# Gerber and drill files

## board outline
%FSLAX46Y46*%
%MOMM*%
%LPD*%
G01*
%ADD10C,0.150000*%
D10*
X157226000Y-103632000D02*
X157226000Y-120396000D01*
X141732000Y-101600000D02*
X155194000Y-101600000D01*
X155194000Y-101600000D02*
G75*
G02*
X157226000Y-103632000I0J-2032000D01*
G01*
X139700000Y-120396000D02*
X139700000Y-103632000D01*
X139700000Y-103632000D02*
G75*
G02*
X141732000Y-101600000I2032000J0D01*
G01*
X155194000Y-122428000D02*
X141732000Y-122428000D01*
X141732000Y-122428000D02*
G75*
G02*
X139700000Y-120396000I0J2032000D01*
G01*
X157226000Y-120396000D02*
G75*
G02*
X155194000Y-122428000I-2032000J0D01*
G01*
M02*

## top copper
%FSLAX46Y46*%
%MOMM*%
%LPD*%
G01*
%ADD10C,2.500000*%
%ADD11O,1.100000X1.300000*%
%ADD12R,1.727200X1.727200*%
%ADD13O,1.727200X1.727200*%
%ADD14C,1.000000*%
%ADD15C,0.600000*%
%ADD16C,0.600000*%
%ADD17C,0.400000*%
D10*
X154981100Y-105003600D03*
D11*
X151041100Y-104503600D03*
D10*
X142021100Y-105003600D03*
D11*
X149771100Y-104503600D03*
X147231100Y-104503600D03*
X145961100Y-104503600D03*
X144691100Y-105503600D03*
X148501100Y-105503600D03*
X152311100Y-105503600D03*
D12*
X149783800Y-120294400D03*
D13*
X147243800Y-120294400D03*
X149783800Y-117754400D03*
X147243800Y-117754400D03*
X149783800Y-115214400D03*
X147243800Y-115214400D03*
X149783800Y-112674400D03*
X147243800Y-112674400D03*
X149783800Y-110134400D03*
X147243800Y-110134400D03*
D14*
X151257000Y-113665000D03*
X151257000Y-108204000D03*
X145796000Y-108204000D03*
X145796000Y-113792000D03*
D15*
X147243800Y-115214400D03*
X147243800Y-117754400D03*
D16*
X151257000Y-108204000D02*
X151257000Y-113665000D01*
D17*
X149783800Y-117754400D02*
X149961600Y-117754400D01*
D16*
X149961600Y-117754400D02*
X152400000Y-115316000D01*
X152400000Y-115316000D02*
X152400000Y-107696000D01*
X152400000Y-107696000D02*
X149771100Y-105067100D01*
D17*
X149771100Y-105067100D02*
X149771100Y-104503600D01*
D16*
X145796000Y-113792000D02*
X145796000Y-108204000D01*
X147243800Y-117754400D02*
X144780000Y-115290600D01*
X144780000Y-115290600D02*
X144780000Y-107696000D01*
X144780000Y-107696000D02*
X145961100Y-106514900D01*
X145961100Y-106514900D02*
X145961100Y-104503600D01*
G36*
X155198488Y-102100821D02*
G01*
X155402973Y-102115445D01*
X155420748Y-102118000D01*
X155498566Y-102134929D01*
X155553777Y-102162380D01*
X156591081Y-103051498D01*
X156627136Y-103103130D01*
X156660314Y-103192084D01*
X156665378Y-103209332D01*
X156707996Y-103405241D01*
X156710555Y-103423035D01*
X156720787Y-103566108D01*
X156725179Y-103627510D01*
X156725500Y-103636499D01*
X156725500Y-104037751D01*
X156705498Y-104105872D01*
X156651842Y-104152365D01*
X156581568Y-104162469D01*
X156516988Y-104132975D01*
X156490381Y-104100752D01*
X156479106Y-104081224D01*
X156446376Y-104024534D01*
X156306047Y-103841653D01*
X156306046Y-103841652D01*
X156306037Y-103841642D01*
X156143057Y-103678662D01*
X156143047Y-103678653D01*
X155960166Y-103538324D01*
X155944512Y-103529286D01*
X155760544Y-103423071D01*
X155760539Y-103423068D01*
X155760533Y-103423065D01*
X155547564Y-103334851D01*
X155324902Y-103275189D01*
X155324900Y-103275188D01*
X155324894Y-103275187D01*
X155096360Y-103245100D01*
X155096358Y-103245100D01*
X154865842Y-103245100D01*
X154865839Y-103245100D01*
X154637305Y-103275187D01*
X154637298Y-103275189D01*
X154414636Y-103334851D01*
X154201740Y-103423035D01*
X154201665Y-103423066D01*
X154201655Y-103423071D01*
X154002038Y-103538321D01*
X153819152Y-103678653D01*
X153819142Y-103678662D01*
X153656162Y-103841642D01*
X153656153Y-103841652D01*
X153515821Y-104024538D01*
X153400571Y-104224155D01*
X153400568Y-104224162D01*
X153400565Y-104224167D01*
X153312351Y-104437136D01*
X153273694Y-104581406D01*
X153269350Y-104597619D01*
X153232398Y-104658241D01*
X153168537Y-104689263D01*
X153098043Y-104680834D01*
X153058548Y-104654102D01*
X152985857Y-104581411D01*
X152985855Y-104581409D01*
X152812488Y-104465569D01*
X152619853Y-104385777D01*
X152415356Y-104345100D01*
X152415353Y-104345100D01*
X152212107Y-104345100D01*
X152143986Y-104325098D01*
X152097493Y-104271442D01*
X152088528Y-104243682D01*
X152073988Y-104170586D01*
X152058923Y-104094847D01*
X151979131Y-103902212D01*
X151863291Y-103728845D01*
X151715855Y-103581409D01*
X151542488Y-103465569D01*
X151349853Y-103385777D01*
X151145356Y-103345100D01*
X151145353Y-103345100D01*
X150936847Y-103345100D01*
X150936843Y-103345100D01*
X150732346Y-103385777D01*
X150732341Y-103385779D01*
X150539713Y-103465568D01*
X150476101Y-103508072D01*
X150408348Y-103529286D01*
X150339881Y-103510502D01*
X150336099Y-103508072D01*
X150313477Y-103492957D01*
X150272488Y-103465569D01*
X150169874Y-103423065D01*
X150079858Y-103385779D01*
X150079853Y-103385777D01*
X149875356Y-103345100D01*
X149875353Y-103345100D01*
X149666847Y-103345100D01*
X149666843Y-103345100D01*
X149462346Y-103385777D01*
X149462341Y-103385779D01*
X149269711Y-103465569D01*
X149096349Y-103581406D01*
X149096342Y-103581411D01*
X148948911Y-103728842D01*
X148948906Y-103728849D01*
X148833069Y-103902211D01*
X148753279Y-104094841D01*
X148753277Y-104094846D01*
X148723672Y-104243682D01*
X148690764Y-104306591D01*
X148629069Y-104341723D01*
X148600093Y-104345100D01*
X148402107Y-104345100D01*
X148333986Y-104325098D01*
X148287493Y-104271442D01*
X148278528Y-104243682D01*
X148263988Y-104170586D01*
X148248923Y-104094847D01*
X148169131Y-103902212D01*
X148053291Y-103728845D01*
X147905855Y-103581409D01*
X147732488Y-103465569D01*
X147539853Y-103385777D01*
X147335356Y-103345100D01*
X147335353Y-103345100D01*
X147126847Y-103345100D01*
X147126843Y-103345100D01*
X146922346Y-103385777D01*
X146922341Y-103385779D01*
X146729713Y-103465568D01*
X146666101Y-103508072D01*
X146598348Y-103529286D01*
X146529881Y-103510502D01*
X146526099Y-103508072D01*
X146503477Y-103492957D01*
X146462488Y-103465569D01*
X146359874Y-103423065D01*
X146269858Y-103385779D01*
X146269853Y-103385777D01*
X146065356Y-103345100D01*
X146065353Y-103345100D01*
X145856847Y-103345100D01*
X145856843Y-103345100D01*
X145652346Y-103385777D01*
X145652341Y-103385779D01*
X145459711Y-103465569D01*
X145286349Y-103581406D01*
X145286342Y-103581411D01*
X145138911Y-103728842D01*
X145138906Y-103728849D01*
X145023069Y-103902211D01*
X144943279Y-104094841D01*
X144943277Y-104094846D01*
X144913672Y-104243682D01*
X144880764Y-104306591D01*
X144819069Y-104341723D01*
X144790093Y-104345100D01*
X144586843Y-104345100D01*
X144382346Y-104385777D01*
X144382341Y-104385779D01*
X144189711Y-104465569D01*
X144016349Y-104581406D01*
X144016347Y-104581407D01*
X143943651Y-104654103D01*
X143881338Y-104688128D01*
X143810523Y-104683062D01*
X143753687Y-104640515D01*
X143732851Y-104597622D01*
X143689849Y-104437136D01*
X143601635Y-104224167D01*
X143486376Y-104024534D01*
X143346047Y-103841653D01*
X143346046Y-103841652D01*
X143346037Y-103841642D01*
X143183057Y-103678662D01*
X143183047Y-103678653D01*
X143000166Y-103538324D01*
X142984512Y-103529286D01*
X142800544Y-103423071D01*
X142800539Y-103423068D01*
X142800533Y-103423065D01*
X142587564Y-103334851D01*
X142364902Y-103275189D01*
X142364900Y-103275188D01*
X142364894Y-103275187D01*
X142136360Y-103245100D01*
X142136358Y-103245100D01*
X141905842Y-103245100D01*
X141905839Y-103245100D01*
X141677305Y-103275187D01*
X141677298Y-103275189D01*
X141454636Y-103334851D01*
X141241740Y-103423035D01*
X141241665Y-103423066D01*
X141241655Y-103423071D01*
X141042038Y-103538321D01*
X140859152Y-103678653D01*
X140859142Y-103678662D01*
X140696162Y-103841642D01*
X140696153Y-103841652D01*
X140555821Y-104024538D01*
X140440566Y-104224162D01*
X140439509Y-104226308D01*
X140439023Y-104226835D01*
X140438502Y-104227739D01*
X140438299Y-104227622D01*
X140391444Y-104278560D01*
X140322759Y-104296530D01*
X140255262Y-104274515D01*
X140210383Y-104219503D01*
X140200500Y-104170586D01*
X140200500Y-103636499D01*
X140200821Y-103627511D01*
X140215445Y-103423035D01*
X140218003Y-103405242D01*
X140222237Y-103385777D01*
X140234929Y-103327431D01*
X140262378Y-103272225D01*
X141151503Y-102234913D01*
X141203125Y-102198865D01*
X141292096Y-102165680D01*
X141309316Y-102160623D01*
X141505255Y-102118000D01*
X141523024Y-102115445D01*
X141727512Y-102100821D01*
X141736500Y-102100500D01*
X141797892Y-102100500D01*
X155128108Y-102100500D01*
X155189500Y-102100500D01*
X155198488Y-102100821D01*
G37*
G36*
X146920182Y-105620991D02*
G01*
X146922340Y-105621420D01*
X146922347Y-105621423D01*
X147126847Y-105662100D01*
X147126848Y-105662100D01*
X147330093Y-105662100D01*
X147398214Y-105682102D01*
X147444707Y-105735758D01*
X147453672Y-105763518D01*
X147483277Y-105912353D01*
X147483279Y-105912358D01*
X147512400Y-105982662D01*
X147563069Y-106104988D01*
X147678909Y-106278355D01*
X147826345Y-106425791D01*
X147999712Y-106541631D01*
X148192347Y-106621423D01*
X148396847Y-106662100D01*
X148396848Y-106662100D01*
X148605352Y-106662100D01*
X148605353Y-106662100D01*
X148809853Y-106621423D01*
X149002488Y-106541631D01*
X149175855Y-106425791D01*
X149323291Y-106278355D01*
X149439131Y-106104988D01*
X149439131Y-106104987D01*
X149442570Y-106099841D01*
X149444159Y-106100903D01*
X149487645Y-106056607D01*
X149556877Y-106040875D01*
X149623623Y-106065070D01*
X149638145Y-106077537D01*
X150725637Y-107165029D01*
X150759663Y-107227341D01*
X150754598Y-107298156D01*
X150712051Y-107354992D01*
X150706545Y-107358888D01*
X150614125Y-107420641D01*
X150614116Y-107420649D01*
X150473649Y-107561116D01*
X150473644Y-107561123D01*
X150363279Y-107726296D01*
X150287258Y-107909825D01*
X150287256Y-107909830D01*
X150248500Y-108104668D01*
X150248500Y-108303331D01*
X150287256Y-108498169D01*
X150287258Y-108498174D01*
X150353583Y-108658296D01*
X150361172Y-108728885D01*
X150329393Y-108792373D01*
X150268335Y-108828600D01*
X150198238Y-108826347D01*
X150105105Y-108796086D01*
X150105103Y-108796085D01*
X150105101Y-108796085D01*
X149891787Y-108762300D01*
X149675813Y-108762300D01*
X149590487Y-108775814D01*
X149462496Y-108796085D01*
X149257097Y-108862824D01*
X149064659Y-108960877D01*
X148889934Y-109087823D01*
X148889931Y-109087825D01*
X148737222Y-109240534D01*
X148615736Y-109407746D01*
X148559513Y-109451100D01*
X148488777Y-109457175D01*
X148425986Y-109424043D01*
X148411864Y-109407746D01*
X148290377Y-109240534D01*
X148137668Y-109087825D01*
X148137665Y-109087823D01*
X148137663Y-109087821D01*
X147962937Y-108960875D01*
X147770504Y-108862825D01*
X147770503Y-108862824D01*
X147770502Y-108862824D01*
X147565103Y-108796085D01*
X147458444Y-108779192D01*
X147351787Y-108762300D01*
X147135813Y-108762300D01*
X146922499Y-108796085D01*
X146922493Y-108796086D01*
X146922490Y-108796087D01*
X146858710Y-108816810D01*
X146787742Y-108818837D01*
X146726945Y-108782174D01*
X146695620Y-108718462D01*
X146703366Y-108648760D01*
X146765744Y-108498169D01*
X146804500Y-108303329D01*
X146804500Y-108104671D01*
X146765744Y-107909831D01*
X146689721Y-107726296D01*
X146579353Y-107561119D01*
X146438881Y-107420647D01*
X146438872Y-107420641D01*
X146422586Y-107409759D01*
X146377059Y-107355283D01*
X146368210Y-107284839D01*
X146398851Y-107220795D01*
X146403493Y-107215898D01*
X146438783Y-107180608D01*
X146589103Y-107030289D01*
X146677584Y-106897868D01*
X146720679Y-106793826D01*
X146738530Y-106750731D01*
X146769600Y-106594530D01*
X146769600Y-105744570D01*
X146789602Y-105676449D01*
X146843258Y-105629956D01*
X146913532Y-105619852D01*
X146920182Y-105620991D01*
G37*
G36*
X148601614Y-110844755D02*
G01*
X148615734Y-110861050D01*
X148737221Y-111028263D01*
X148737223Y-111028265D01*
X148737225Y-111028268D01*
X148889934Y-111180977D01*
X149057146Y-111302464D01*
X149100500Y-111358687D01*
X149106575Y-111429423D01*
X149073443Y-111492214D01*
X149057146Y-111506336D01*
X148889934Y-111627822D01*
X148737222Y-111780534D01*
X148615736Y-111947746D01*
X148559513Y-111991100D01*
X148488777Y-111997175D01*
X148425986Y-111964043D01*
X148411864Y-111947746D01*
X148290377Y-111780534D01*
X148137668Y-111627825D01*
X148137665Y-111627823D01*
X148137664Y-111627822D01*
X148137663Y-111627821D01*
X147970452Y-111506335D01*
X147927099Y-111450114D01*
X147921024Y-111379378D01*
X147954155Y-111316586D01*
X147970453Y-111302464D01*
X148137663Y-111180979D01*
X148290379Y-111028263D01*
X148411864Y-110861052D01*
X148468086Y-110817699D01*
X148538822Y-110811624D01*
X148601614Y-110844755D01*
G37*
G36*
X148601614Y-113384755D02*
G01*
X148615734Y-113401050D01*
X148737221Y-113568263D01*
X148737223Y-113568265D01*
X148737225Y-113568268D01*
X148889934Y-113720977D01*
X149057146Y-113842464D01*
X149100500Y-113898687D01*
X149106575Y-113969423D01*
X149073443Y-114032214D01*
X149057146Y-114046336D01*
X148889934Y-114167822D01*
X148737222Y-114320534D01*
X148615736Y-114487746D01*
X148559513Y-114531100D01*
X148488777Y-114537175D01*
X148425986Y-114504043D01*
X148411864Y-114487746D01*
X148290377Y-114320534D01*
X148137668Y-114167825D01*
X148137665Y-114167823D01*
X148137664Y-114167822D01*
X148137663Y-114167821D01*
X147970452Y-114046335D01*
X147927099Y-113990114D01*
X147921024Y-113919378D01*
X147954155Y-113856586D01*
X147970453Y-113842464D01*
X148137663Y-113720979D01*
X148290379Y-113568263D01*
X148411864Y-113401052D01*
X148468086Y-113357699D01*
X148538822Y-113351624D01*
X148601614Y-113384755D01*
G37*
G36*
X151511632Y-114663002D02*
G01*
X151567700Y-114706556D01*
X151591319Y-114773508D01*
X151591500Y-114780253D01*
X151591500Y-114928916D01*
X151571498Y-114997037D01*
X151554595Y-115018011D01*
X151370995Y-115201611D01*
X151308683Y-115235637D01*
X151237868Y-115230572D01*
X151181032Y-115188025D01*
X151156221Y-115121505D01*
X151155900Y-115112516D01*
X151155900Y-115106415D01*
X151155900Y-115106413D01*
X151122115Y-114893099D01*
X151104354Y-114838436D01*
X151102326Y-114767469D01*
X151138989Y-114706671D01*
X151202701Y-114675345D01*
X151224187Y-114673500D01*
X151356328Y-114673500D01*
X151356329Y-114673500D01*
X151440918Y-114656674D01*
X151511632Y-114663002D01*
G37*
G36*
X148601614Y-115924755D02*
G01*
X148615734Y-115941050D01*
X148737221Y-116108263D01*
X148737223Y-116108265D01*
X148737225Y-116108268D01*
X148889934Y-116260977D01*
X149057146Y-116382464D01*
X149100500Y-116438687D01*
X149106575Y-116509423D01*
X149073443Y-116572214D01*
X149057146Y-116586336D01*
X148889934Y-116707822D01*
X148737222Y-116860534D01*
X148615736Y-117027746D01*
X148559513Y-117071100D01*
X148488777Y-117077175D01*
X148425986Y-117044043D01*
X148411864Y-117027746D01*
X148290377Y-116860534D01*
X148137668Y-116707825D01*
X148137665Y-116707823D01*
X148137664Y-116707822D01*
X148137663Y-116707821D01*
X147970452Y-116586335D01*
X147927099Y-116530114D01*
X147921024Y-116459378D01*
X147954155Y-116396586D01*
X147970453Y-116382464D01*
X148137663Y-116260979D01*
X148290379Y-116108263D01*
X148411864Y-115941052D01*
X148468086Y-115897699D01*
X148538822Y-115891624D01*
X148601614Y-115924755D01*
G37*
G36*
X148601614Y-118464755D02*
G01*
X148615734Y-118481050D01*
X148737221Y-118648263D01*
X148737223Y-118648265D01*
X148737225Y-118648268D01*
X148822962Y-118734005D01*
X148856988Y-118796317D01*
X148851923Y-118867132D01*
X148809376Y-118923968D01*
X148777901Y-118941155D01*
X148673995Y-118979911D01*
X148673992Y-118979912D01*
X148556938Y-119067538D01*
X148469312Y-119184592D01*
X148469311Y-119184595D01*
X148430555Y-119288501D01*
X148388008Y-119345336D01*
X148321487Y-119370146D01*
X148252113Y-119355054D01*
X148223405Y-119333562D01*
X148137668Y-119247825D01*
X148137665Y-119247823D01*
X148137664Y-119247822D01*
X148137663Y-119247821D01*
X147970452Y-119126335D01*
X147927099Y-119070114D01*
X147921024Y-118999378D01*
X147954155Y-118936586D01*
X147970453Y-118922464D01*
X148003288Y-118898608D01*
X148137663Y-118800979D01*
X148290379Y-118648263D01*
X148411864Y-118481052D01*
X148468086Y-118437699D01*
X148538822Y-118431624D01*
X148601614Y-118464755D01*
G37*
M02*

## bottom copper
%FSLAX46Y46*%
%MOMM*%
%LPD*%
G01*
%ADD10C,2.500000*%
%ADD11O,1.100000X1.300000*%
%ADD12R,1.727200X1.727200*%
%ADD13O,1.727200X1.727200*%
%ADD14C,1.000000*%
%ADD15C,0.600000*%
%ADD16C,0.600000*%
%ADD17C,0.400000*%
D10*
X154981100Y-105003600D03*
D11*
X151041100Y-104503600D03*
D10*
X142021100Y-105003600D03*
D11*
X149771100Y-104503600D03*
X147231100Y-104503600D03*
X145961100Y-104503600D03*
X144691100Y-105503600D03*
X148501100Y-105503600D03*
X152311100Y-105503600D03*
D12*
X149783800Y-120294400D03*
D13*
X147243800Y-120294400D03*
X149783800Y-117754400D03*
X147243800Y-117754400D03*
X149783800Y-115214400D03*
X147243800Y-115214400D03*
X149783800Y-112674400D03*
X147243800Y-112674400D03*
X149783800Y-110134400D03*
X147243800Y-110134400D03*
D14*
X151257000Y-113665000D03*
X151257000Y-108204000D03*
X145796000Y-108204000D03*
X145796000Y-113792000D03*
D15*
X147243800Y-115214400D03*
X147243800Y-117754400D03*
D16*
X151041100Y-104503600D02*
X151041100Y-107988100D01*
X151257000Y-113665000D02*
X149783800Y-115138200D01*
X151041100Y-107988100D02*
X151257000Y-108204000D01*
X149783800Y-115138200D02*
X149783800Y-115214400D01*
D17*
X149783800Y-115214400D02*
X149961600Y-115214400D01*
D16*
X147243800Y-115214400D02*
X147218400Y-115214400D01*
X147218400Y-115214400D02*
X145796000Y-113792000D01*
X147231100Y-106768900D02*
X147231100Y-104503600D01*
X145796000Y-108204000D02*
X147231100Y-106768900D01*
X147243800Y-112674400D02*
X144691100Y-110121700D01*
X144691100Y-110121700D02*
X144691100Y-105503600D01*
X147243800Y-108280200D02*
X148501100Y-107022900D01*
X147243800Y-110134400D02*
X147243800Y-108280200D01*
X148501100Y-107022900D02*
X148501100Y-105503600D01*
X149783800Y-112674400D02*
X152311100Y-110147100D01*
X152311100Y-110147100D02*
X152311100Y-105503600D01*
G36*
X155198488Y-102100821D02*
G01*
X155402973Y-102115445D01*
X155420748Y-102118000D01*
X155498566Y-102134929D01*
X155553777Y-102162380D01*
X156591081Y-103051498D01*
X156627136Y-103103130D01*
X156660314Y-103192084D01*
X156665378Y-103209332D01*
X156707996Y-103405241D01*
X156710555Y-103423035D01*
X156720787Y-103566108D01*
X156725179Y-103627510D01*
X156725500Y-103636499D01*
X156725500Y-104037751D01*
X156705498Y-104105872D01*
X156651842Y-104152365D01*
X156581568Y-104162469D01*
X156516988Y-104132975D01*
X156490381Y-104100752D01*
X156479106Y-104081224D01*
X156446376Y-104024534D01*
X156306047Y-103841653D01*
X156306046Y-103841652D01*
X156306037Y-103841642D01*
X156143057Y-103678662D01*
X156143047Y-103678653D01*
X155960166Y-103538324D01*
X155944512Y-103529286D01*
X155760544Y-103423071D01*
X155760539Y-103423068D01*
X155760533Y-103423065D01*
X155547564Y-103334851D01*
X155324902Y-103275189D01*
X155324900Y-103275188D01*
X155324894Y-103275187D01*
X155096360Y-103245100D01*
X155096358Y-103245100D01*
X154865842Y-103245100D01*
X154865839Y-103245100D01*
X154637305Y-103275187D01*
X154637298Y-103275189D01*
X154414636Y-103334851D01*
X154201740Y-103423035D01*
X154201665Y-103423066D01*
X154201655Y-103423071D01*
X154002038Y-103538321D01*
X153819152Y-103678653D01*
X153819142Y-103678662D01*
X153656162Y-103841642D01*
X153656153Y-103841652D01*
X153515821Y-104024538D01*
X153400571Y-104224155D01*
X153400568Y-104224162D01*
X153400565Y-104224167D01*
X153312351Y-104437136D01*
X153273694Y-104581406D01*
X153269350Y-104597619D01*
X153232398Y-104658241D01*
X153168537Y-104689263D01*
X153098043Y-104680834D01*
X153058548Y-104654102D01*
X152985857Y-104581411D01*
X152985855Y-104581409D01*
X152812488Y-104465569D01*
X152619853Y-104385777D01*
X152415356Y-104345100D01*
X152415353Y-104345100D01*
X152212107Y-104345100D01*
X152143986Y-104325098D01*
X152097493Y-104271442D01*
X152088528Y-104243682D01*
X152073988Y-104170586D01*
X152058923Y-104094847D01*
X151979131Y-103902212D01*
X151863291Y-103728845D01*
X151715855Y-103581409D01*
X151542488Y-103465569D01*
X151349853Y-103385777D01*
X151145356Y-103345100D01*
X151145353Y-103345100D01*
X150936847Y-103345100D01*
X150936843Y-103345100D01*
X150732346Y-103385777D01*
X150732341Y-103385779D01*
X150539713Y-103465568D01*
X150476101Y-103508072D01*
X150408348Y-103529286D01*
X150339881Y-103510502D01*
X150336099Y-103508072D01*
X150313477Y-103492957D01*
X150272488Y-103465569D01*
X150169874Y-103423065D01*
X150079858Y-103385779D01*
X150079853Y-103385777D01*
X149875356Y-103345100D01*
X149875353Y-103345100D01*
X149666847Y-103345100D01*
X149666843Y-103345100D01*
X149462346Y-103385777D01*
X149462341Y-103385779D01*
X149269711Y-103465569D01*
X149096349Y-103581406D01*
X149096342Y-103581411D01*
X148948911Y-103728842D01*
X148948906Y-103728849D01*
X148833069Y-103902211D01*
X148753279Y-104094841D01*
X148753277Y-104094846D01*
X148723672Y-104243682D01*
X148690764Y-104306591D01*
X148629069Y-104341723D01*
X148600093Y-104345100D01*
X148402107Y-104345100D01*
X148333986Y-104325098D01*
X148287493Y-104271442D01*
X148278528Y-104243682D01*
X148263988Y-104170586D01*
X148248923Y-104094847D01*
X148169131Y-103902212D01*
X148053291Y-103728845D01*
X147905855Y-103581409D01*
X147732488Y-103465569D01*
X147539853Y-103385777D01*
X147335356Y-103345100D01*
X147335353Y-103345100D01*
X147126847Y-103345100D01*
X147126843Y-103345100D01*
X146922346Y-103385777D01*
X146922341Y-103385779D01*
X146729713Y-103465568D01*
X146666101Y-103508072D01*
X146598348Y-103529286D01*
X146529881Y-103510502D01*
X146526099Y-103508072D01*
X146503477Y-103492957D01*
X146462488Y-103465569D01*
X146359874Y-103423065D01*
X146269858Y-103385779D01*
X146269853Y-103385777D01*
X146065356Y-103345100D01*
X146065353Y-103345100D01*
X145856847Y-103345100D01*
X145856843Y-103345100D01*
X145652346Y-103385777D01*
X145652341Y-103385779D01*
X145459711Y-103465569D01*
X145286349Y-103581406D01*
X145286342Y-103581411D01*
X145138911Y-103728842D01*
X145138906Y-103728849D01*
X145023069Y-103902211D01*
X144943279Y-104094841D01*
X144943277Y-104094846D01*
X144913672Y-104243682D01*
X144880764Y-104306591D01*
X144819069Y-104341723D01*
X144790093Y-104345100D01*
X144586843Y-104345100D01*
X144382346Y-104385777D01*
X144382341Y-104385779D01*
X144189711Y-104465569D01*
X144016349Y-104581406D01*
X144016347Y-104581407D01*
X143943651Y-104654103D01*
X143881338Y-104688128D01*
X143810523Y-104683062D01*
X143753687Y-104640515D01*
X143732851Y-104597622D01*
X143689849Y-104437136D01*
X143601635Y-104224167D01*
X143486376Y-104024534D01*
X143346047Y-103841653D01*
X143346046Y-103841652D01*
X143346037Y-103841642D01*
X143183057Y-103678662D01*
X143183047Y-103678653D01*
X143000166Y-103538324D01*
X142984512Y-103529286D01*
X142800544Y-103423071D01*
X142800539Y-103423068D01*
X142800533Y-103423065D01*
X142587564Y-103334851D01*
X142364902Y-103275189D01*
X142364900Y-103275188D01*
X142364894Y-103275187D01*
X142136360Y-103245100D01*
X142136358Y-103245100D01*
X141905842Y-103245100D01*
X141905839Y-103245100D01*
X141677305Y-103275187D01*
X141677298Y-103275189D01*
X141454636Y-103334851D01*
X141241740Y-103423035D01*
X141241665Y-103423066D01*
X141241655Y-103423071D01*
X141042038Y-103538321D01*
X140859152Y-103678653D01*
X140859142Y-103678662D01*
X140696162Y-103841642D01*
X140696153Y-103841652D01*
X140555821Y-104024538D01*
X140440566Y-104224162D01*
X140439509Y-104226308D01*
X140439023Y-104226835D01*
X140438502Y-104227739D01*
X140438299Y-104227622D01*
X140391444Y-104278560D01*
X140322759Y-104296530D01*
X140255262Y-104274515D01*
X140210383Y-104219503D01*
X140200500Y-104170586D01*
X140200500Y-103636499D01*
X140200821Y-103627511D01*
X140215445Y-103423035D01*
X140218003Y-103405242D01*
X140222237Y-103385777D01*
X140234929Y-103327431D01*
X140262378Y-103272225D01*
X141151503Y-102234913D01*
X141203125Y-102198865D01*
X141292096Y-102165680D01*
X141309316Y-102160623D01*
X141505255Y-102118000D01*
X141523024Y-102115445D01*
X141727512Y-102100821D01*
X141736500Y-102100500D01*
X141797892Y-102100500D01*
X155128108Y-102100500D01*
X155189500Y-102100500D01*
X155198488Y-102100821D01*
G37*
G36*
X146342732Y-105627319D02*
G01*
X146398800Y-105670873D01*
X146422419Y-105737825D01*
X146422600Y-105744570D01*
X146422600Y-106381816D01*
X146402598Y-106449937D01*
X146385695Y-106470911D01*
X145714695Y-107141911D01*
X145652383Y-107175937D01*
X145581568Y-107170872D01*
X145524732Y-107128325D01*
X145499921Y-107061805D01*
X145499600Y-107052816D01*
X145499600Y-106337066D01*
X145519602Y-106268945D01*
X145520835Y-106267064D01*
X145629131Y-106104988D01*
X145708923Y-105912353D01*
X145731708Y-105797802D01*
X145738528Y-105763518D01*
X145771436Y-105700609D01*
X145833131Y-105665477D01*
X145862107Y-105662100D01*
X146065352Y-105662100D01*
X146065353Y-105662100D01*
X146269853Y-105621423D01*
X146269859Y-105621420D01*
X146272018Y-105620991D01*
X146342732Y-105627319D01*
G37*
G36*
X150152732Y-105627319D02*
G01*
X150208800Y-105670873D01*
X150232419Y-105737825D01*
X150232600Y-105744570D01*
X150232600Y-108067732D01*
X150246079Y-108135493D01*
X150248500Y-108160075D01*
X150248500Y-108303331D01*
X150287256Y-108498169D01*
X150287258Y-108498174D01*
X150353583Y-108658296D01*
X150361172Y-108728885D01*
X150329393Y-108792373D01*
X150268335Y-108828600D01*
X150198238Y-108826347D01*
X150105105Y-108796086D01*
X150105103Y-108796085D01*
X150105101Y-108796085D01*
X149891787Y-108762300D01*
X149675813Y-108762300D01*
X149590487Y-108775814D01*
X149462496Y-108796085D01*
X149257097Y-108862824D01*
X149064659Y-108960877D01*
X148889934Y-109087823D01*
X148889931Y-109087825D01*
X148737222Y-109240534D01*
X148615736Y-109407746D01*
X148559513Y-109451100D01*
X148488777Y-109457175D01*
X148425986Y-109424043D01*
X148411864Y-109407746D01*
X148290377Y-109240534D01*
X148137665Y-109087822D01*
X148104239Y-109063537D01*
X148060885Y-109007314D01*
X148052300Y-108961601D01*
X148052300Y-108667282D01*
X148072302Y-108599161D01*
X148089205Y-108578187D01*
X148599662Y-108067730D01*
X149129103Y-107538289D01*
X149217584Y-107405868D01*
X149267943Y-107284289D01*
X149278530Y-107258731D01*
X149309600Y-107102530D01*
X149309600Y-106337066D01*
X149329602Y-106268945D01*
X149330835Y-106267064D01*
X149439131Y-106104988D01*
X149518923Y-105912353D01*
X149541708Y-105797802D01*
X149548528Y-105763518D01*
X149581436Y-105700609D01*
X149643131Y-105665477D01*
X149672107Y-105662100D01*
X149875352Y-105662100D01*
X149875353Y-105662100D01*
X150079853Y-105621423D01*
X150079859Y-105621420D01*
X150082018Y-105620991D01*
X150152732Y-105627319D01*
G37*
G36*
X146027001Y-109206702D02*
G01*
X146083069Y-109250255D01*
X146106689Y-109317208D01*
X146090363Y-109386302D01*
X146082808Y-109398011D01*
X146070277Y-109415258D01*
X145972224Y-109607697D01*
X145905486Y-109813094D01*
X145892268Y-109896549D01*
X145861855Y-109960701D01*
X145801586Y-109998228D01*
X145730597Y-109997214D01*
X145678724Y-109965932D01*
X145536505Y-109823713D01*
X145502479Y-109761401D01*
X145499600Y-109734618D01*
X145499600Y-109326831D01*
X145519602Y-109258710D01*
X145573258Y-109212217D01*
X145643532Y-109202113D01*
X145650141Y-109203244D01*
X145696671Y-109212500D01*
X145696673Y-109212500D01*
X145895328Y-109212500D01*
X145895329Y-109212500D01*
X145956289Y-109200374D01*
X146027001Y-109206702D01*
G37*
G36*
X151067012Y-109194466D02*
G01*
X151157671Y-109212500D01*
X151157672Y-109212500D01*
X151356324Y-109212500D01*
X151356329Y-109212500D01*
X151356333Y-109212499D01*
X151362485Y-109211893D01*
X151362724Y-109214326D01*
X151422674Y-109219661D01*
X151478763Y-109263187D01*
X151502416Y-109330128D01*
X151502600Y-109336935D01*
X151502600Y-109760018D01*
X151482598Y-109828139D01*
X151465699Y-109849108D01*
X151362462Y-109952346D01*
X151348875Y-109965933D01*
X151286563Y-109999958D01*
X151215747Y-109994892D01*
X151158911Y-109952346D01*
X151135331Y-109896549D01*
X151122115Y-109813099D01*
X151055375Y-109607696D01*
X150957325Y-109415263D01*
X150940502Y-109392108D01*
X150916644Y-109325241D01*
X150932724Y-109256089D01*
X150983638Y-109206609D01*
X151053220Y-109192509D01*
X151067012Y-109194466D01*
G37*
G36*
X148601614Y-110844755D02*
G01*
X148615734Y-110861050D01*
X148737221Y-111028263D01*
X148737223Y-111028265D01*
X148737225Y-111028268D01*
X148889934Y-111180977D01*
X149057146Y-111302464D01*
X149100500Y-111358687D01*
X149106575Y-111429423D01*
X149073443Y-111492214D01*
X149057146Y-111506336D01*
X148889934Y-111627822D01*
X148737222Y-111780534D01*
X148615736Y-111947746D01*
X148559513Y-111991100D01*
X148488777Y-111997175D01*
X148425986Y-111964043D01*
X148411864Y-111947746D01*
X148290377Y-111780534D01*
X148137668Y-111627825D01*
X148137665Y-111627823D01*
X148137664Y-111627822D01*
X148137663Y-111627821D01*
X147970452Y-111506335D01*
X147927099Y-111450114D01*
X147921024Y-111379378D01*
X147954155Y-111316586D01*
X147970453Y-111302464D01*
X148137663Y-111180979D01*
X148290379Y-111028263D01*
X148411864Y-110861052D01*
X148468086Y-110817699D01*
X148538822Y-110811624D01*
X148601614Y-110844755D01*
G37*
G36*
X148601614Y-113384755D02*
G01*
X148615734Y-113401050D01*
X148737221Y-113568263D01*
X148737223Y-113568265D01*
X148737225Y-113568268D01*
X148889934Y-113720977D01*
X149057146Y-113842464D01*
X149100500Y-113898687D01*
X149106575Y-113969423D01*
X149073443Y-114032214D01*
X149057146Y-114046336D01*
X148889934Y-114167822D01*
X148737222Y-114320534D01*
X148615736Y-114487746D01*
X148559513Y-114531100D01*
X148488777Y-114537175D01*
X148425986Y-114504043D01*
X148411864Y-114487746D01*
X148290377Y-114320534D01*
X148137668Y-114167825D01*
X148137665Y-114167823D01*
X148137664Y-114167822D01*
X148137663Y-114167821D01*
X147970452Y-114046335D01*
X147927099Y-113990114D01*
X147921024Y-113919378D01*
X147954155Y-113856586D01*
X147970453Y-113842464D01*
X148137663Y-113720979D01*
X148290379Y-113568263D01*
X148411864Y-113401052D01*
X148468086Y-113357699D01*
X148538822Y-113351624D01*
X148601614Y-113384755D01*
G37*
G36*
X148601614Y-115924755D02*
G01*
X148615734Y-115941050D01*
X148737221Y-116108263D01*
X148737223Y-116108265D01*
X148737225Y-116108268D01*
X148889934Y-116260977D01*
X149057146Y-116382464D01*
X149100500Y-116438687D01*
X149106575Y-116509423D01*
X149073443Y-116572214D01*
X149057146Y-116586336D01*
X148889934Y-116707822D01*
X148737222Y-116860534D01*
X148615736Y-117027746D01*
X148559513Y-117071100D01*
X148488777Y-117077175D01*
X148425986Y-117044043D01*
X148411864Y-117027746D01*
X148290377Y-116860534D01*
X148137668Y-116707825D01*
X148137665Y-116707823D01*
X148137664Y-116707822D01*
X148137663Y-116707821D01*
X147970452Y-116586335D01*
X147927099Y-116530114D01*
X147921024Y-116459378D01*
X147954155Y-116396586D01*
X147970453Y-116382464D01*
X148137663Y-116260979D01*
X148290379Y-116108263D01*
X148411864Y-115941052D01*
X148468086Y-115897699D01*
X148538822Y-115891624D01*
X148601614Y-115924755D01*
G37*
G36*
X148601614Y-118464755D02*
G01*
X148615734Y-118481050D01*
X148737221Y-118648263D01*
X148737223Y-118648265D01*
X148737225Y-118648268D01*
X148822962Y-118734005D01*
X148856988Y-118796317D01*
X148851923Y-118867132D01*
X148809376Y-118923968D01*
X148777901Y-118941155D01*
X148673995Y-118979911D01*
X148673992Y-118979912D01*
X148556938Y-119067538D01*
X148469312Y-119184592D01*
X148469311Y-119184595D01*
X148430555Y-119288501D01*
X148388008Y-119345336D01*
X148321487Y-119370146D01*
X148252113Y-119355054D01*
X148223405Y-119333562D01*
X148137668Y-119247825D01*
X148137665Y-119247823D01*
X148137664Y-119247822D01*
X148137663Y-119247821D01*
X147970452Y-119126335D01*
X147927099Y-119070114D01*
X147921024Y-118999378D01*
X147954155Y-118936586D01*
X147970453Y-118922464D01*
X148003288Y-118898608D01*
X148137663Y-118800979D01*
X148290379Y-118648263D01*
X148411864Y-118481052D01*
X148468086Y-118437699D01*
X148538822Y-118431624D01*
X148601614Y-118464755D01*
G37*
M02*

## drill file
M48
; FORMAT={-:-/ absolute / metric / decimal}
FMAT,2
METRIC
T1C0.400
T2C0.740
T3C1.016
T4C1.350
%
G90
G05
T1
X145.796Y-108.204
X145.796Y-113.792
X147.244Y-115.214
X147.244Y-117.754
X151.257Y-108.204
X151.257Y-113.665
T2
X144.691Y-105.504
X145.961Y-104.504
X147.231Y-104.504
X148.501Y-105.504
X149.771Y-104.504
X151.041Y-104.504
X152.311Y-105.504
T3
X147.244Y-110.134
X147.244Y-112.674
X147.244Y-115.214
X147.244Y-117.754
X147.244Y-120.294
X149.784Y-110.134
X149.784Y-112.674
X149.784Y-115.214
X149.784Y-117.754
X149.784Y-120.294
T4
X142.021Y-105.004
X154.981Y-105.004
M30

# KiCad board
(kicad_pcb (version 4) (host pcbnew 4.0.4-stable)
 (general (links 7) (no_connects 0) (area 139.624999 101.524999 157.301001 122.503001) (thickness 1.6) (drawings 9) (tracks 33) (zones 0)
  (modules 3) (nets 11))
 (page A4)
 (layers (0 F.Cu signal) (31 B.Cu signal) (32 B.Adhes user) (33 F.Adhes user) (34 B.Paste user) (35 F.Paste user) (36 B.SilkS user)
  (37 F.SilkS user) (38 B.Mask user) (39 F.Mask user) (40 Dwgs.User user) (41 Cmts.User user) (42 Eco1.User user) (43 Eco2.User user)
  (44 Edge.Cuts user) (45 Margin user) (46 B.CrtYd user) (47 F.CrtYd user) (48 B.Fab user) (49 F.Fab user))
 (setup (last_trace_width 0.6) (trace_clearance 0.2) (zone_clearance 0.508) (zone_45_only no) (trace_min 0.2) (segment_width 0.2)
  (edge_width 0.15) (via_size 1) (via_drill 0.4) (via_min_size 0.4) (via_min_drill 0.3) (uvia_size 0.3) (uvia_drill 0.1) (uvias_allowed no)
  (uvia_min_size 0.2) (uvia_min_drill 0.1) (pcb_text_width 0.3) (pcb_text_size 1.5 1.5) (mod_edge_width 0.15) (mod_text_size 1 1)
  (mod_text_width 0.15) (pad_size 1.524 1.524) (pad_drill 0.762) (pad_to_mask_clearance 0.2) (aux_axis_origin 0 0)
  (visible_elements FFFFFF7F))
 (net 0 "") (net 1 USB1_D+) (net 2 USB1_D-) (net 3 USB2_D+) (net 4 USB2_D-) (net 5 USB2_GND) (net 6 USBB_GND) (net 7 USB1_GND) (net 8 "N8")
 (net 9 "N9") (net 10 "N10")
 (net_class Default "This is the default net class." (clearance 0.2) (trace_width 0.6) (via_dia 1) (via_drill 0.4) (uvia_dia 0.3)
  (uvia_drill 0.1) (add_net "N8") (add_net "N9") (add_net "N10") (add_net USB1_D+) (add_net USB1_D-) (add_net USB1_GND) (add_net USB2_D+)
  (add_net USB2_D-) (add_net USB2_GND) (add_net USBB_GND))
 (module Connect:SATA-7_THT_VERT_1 (layer F.Cu) (at 148.5011 105.0036)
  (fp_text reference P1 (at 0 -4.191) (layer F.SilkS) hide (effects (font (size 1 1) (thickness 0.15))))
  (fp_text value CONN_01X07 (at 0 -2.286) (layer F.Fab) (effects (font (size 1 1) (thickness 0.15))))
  (pad 9 thru_hole circle (at 6.48 0) (size 2.5 2.5) (drill 1.35) (layers *.Cu *.Mask F.SilkS))
  (pad 2 thru_hole oval (at 2.54 -0.5) (size 1.1 1.3) (drill 0.74) (layers *.Cu *.Mask F.SilkS) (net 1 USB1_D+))
  (pad 8 thru_hole circle (at -6.48 0) (size 2.5 2.5) (drill 1.35) (layers *.Cu *.Mask F.SilkS))
  (pad 3 thru_hole oval (at 1.27 -0.5) (size 1.1 1.3) (drill 0.74) (layers *.Cu *.Mask F.SilkS) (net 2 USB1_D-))
  (pad 5 thru_hole oval (at -1.27 -0.5) (size 1.1 1.3) (drill 0.74) (layers *.Cu *.Mask F.SilkS) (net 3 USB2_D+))
  (pad 6 thru_hole oval (at -2.54 -0.5) (size 1.1 1.3) (drill 0.74) (layers *.Cu *.Mask F.SilkS) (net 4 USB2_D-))
  (pad 7 thru_hole oval (at -3.81 0.5) (size 1.1 1.3) (drill 0.74) (layers *.Cu *.Mask F.SilkS) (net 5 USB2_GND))
  (pad 4 thru_hole oval (at 0 0.5) (size 1.1 1.3) (drill 0.74) (layers *.Cu *.Mask F.SilkS) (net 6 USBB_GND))
  (pad 1 thru_hole oval (at 3.81 0.5) (size 1.1 1.3) (drill 0.74) (layers *.Cu *.Mask F.SilkS) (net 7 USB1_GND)))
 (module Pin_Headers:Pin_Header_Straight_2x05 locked (layer F.Cu) (at 149.7838 120.2944 180)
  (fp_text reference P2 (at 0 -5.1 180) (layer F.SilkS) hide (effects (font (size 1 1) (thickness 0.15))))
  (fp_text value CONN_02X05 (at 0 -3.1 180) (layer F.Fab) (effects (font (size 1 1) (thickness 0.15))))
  (pad 1 thru_hole rect (at 0 0 180) (size 1.7272 1.7272) (drill 1.016) (layers *.Cu *.Mask F.SilkS) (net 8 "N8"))
  (pad 2 thru_hole oval (at 2.54 0 180) (size 1.7272 1.7272) (drill 1.016) (layers *.Cu *.Mask F.SilkS) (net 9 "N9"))
  (pad 3 thru_hole oval (at 0 2.54 180) (size 1.7272 1.7272) (drill 1.016) (layers *.Cu *.Mask F.SilkS) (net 2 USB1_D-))
  (pad 4 thru_hole oval (at 2.54 2.54 180) (size 1.7272 1.7272) (drill 1.016) (layers *.Cu *.Mask F.SilkS) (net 4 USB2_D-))
  (pad 5 thru_hole oval (at 0 5.08 180) (size 1.7272 1.7272) (drill 1.016) (layers *.Cu *.Mask F.SilkS) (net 1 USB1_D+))
  (pad 6 thru_hole oval (at 2.54 5.08 180) (size 1.7272 1.7272) (drill 1.016) (layers *.Cu *.Mask F.SilkS) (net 3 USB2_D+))
  (pad 7 thru_hole oval (at 0 7.62 180) (size 1.7272 1.7272) (drill 1.016) (layers *.Cu *.Mask F.SilkS) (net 7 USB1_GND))
  (pad 8 thru_hole oval (at 2.54 7.62 180) (size 1.7272 1.7272) (drill 1.016) (layers *.Cu *.Mask F.SilkS) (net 5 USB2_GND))
  (pad 9 thru_hole oval (at 0 10.16 180) (size 1.7272 1.7272) (drill 1.016) (layers *.Cu *.Mask F.SilkS) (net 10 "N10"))
  (pad 10 thru_hole oval (at 2.54 10.16 180) (size 1.7272 1.7272) (drill 1.016) (layers *.Cu *.Mask F.SilkS) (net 6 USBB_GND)))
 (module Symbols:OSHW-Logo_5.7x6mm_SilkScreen (layer F.Cu) (at 142.875 117.221)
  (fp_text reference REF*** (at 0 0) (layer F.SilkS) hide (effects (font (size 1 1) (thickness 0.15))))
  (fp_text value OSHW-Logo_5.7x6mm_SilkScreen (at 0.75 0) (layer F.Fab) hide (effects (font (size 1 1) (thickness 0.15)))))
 (gr_line (start 157.226 103.632) (end 157.226 120.396) (angle 90) (layer Edge.Cuts) (width 0.15))
 (gr_line (start 141.732 101.6) (end 155.194 101.6) (angle 90) (layer Edge.Cuts) (width 0.15))
 (gr_arc (start 155.194 103.632) (end 155.194 101.6) (angle 90) (layer Edge.Cuts) (width 0.15))
 (gr_line (start 139.7 120.396) (end 139.7 103.632) (angle 90) (layer Edge.Cuts) (width 0.15))
 (gr_arc (start 141.732 103.632) (end 139.7 103.632) (angle 90) (layer Edge.Cuts) (width 0.15))
 (gr_line (start 155.194 122.428) (end 141.732 122.428) (angle 90) (layer Edge.Cuts) (width 0.15))
 (gr_arc (start 141.732 120.396) (end 141.732 122.428) (angle 90) (layer Edge.Cuts) (width 0.15))
 (gr_arc (start 155.194 120.396) (end 157.226 120.396) (angle 90) (layer Edge.Cuts) (width 0.15))
 (segment (start 151.0411 104.5036) (end 151.0411 107.9881) (width 0.6) (layer B.Cu) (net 1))
 (segment (start 151.257 113.665) (end 149.7838 115.1382) (width 0.6) (layer B.Cu) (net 1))
 (via (at 151.257 113.665) (size 1) (drill 0.4) (layers F.Cu B.Cu) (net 1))
 (segment (start 151.257 108.204) (end 151.257 113.665) (width 0.6) (layer F.Cu) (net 1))
 (via (at 151.257 108.204) (size 1) (drill 0.4) (layers F.Cu B.Cu) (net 1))
 (segment (start 151.0411 107.9881) (end 151.257 108.204) (width 0.6) (layer B.Cu) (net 1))
 (segment (start 149.7838 115.1382) (end 149.7838 115.2144) (width 0.6) (layer B.Cu) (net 1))
 (segment (start 149.7838 115.2144) (end 149.9616 115.2144) (width 0.4) (layer B.Cu) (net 1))
 (segment (start 149.7838 117.7544) (end 149.9616 117.7544) (width 0.4) (layer F.Cu) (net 2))
 (segment (start 149.9616 117.7544) (end 152.4 115.316) (width 0.6) (layer F.Cu) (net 2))
 (segment (start 152.4 115.316) (end 152.4 107.696) (width 0.6) (layer F.Cu) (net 2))
 (segment (start 152.4 107.696) (end 149.7711 105.0671) (width 0.6) (layer F.Cu) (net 2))
 (segment (start 149.7711 105.0671) (end 149.7711 104.5036) (width 0.4) (layer F.Cu) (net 2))
 (segment (start 147.2438 115.2144) (end 147.2184 115.2144) (width 0.6) (layer B.Cu) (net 3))
 (segment (start 147.2184 115.2144) (end 145.796 113.792) (width 0.6) (layer B.Cu) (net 3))
 (segment (start 147.2311 106.7689) (end 147.2311 104.5036) (width 0.6) (layer B.Cu) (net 3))
 (segment (start 145.796 108.204) (end 147.2311 106.7689) (width 0.6) (layer B.Cu) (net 3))
 (via (at 145.796 108.204) (size 1) (drill 0.4) (layers F.Cu B.Cu) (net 3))
 (segment (start 145.796 113.792) (end 145.796 108.204) (width 0.6) (layer F.Cu) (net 3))
 (via (at 145.796 113.792) (size 1) (drill 0.4) (layers F.Cu B.Cu) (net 3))
 (via (at 147.2438 115.2144) (size 0.6) (drill 0.4) (layers F.Cu B.Cu) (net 3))
 (via (at 147.2438 117.7544) (size 0.6) (drill 0.4) (layers F.Cu B.Cu) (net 4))
 (segment (start 147.2438 117.7544) (end 144.78 115.2906) (width 0.6) (layer F.Cu) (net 4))
 (segment (start 144.78 115.2906) (end 144.78 107.696) (width 0.6) (layer F.Cu) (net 4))
 (segment (start 144.78 107.696) (end 145.9611 106.5149) (width 0.6) (layer F.Cu) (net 4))
 (segment (start 145.9611 106.5149) (end 145.9611 104.5036) (width 0.6) (layer F.Cu) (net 4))
 (segment (start 147.2438 112.6744) (end 144.6911 110.1217) (width 0.6) (layer B.Cu) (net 5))
 (segment (start 144.6911 110.1217) (end 144.6911 105.5036) (width 0.6) (layer B.Cu) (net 5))
 (segment (start 147.2438 108.2802) (end 148.5011 107.0229) (width 0.6) (layer B.Cu) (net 6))
 (segment (start 147.2438 110.1344) (end 147.2438 108.2802) (width 0.6) (layer B.Cu) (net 6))
 (segment (start 148.5011 107.0229) (end 148.5011 105.5036) (width 0.6) (layer B.Cu) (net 6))
 (segment (start 149.7838 112.6744) (end 152.3111 110.1471) (width 0.6) (layer B.Cu) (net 7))
 (segment (start 152.3111 110.1471) (end 152.3111 105.5036) (width 0.6) (layer B.Cu) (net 7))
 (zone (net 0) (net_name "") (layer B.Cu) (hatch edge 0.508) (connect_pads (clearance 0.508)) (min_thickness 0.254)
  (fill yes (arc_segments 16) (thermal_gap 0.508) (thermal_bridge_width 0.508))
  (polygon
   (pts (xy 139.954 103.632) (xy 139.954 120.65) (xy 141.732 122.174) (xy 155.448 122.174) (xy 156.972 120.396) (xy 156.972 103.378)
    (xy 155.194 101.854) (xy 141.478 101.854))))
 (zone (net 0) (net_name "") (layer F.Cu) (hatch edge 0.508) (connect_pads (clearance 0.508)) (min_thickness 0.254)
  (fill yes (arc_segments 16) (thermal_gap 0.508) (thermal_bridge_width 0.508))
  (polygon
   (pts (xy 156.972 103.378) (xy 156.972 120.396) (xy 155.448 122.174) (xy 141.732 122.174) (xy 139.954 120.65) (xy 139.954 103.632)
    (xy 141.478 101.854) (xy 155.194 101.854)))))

